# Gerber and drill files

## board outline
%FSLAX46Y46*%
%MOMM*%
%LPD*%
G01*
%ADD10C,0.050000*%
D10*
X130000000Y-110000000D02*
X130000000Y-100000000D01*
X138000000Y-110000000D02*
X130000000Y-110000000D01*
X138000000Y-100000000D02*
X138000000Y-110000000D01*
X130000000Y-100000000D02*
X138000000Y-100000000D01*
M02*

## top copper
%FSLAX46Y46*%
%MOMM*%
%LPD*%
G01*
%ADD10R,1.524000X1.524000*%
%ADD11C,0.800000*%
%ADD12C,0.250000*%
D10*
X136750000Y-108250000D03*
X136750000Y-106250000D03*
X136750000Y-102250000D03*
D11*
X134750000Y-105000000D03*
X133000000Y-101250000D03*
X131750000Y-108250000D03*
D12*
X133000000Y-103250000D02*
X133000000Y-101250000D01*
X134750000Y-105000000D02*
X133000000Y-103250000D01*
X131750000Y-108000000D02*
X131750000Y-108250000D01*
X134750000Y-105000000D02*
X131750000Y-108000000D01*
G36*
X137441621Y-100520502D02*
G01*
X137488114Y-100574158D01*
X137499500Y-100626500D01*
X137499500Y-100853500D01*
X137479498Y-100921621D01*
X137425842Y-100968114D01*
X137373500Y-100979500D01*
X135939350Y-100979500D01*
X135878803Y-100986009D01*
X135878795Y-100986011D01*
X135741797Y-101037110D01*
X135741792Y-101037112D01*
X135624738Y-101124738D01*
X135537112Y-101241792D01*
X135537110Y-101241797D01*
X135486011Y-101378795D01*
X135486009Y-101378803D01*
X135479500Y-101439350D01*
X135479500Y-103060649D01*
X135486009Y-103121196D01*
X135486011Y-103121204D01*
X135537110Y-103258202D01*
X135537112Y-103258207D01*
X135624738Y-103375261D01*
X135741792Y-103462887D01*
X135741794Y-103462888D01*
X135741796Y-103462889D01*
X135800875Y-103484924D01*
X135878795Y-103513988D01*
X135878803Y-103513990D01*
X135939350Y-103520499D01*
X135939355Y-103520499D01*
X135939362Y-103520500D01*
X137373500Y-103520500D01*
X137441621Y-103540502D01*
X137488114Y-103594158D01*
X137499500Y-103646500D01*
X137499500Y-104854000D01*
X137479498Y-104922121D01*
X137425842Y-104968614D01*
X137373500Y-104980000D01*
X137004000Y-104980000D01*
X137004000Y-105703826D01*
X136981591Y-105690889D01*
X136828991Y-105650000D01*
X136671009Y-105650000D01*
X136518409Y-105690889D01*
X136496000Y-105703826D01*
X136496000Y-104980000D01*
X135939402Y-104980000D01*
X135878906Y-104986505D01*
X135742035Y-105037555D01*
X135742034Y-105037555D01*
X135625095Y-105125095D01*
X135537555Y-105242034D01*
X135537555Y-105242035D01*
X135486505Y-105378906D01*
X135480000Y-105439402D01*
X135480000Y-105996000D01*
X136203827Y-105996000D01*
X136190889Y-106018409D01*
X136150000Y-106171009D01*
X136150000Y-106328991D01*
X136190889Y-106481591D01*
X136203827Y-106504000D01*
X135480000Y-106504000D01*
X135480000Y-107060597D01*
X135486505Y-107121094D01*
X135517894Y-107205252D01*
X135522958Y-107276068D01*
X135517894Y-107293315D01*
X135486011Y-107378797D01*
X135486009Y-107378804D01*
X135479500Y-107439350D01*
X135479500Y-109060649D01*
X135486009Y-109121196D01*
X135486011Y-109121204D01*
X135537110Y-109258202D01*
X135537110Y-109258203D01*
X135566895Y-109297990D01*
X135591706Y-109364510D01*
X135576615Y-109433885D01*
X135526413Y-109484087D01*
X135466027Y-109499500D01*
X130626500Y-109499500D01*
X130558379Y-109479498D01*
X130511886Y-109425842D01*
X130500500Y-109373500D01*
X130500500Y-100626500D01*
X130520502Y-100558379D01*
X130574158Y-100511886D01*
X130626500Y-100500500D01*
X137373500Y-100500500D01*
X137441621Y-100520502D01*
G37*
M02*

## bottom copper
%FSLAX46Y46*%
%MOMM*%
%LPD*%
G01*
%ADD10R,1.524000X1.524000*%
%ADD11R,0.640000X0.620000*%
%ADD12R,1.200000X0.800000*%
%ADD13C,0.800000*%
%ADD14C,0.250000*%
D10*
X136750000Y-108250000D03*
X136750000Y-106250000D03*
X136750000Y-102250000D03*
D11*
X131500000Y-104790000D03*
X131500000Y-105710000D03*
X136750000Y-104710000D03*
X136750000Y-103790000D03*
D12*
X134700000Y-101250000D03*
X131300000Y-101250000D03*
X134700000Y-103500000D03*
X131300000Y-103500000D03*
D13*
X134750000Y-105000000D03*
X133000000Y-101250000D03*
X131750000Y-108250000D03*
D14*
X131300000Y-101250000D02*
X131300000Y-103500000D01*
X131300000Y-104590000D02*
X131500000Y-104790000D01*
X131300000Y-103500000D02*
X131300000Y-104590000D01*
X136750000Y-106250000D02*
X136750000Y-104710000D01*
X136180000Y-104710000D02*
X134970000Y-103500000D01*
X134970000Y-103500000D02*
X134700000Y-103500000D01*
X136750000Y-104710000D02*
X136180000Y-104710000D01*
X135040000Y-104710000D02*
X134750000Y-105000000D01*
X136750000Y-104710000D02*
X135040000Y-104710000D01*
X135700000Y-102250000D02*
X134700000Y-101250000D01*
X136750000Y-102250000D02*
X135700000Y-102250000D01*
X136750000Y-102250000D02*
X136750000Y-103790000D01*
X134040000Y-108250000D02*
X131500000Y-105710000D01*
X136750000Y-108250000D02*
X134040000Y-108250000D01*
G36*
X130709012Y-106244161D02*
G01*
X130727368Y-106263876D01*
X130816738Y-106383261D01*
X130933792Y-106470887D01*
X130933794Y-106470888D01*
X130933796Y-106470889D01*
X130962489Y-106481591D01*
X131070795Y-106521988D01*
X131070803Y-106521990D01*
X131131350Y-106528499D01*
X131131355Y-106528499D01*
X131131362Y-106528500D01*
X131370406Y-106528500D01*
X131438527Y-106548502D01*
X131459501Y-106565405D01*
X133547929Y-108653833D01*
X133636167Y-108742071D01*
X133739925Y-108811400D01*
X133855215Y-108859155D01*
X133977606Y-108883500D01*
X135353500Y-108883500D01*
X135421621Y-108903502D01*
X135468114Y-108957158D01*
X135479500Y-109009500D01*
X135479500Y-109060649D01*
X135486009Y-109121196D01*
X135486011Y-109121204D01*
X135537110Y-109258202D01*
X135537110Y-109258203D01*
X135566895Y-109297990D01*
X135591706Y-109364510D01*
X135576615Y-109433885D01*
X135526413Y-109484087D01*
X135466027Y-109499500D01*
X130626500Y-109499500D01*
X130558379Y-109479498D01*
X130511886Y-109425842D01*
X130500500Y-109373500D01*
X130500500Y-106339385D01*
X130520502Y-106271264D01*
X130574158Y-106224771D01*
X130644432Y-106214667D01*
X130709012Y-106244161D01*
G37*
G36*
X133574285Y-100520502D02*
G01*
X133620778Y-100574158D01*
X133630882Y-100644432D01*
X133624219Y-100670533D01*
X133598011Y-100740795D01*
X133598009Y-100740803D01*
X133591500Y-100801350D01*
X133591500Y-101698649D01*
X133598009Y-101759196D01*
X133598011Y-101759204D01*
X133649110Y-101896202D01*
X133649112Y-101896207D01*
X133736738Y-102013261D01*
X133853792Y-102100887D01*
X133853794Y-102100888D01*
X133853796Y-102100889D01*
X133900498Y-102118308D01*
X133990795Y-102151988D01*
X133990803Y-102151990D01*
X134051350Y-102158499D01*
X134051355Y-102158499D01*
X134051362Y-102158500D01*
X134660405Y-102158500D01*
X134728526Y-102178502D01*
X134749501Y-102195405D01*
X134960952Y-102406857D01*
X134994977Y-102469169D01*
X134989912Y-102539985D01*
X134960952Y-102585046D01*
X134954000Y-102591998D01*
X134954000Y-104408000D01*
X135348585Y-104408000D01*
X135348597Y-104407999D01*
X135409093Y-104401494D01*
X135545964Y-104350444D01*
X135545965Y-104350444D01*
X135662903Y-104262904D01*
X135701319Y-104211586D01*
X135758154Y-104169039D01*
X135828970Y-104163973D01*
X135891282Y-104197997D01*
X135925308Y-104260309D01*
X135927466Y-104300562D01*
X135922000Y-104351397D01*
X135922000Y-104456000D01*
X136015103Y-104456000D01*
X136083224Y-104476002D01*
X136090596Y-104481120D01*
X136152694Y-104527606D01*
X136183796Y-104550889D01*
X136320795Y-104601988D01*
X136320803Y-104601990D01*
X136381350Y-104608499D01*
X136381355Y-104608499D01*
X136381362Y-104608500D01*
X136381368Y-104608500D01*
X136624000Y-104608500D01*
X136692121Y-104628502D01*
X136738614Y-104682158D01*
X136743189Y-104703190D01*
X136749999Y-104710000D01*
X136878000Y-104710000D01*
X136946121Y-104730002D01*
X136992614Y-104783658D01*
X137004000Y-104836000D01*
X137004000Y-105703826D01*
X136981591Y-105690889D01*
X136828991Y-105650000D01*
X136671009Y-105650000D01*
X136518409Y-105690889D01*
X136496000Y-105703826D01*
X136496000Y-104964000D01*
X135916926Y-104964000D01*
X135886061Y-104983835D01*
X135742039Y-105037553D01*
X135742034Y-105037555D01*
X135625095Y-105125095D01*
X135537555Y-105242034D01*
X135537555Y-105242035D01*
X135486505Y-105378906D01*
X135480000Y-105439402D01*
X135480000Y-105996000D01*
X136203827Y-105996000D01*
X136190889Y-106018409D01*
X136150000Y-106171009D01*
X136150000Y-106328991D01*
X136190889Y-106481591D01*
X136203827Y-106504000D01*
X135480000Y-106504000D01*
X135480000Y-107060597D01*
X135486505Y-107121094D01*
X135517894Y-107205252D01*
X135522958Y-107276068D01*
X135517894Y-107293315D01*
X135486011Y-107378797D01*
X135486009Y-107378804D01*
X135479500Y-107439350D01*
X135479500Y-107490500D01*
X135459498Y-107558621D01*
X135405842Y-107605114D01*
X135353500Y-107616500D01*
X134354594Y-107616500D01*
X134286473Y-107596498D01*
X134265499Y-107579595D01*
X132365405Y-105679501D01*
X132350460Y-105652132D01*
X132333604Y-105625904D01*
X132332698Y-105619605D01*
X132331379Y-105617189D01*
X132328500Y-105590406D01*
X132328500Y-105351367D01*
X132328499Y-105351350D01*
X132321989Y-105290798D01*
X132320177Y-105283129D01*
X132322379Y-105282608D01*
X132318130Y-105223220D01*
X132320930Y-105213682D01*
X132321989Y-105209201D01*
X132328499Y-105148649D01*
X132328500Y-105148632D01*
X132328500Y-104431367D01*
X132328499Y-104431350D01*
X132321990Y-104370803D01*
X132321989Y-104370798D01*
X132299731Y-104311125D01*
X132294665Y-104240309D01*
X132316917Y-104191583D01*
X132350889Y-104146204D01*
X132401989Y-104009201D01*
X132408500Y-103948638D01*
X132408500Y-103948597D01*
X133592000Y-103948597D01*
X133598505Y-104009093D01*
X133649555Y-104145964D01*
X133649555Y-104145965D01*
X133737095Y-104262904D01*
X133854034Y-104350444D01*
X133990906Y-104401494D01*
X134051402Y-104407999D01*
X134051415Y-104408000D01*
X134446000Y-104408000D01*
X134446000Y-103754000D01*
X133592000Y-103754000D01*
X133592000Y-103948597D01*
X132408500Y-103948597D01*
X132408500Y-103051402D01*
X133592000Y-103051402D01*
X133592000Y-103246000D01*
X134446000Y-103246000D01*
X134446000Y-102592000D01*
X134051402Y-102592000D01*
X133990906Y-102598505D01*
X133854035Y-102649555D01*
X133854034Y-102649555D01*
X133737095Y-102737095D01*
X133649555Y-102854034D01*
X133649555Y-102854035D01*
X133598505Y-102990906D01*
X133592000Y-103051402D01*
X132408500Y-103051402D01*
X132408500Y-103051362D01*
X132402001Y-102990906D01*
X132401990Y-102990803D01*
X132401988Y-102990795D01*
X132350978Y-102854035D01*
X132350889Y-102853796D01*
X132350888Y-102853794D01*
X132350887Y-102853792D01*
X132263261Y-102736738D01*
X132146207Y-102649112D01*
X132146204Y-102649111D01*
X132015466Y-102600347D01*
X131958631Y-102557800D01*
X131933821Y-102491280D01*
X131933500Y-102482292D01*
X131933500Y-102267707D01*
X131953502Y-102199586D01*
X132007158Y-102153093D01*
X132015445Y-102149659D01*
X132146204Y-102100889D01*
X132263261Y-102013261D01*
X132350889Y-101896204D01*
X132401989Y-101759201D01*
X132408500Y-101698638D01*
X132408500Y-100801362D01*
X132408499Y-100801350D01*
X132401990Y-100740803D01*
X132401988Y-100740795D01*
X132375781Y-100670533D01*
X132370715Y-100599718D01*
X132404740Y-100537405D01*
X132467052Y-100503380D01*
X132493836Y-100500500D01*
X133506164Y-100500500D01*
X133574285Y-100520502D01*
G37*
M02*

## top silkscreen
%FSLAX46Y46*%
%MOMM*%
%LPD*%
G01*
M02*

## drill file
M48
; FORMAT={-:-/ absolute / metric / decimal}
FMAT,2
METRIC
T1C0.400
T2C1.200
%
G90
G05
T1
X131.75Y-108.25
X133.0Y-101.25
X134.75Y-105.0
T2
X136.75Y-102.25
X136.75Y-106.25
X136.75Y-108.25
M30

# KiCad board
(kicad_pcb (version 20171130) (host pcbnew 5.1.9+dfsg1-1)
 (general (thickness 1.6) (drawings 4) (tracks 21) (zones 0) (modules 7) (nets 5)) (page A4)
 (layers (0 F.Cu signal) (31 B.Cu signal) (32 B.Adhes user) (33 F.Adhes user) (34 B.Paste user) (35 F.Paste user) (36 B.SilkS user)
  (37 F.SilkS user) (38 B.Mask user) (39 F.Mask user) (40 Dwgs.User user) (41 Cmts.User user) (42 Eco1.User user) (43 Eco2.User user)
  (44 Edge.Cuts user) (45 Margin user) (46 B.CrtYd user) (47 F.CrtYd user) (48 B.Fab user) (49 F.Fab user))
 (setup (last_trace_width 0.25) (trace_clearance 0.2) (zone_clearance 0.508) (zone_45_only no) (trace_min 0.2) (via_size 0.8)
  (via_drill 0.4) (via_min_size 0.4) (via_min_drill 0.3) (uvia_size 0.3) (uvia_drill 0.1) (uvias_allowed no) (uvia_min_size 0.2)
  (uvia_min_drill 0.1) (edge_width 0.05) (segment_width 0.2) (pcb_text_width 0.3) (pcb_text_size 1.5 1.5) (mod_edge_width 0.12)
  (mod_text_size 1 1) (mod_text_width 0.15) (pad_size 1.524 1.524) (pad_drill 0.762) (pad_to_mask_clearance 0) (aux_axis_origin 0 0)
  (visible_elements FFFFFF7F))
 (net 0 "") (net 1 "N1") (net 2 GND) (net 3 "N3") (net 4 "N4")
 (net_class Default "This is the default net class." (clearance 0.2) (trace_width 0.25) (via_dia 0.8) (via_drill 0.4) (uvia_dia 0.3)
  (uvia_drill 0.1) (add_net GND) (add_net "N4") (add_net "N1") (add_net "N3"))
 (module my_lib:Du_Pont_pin (layer B.Cu) (at 136.75 108.25)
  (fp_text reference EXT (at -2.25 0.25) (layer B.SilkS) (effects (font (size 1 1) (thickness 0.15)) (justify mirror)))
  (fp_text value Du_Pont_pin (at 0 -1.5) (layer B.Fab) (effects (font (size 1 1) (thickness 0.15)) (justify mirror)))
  (pad 1 thru_hole rect (at 0 0) (size 1.524 1.524) (drill 1.2) (layers *.Cu *.Mask) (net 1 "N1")))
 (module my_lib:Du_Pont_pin (layer B.Cu) (at 136.75 106.25)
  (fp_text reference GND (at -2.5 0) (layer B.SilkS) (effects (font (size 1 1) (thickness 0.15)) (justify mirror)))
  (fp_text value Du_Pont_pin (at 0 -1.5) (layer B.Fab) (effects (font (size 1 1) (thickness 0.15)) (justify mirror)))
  (pad 1 thru_hole rect (at 0 0) (size 1.524 1.524) (drill 1.2) (layers *.Cu *.Mask) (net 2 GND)))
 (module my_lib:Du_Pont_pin (layer B.Cu) (at 136.75 102.25)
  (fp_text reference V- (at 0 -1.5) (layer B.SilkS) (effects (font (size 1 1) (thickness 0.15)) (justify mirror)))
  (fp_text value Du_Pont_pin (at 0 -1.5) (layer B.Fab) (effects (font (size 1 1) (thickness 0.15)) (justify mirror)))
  (pad 1 thru_hole rect (at 0 0) (size 1.524 1.524) (drill 1.2) (layers *.Cu *.Mask) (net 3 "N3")))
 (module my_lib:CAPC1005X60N (layer B.Cu) (at 131.5 105.25 270)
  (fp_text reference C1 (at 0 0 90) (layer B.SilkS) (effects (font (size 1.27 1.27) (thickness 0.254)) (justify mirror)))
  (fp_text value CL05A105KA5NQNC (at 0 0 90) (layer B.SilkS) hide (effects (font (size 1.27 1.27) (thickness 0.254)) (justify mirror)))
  (pad 1 smd rect (at -0.46 0 270) (size 0.62 0.64) (layers B.Cu B.Paste B.Mask) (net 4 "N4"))
  (pad 2 smd rect (at 0.46 0 270) (size 0.62 0.64) (layers B.Cu B.Paste B.Mask) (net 1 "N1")))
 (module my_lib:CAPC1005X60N (layer B.Cu) (at 136.75 104.25 270)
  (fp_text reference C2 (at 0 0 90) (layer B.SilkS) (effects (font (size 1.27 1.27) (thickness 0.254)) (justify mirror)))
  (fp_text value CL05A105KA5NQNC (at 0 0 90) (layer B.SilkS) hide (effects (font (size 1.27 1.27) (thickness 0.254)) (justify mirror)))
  (pad 2 smd rect (at 0.46 0 270) (size 0.62 0.64) (layers B.Cu B.Paste B.Mask) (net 2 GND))
  (pad 1 smd rect (at -0.46 0 270) (size 0.62 0.64) (layers B.Cu B.Paste B.Mask) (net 3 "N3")))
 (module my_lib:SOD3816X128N (layer B.Cu) (at 133 101.25)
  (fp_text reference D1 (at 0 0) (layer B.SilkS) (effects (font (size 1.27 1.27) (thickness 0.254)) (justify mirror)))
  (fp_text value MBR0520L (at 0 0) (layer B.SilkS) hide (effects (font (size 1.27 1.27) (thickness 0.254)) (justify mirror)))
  (pad 2 smd rect (at 1.7 0 270) (size 0.8 1.2) (layers B.Cu B.Paste B.Mask) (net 3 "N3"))
  (pad 1 smd rect (at -1.7 0 270) (size 0.8 1.2) (layers B.Cu B.Paste B.Mask) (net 4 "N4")))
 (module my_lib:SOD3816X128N (layer B.Cu) (at 133 103.5 180)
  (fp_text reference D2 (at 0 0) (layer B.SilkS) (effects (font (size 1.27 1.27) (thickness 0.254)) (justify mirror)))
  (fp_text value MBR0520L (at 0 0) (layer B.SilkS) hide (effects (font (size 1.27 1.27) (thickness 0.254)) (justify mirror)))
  (pad 1 smd rect (at -1.7 0 90) (size 0.8 1.2) (layers B.Cu B.Paste B.Mask) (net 2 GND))
  (pad 2 smd rect (at 1.7 0 90) (size 0.8 1.2) (layers B.Cu B.Paste B.Mask) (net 4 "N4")))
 (gr_line (start 130 110) (end 130 100) (layer Edge.Cuts) (width 0.05))
 (gr_line (start 138 110) (end 130 110) (layer Edge.Cuts) (width 0.05))
 (gr_line (start 138 100) (end 138 110) (layer Edge.Cuts) (width 0.05))
 (gr_line (start 130 100) (end 138 100) (layer Edge.Cuts) (width 0.05))
 (segment (start 131.3 101.25) (end 131.3 103.5) (width 0.25) (layer B.Cu) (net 4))
 (segment (start 131.3 104.59) (end 131.5 104.79) (width 0.25) (layer B.Cu) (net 4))
 (segment (start 131.3 103.5) (end 131.3 104.59) (width 0.25) (layer B.Cu) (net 4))
 (segment (start 136.75 106.25) (end 136.75 104.71) (width 0.25) (layer B.Cu) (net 2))
 (segment (start 136.18 104.71) (end 134.97 103.5) (width 0.25) (layer B.Cu) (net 2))
 (segment (start 134.97 103.5) (end 134.7 103.5) (width 0.25) (layer B.Cu) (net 2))
 (segment (start 136.75 104.71) (end 136.18 104.71) (width 0.25) (layer B.Cu) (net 2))
 (via (at 134.75 105) (size 0.8) (drill 0.4) (layers F.Cu B.Cu) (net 2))
 (segment (start 135.04 104.71) (end 134.75 105) (width 0.25) (layer B.Cu) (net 2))
 (segment (start 136.75 104.71) (end 135.04 104.71) (width 0.25) (layer B.Cu) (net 2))
 (via (at 133 101.25) (size 0.8) (drill 0.4) (layers F.Cu B.Cu) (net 2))
 (segment (start 133 103.25) (end 133 101.25) (width 0.25) (layer F.Cu) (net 2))
 (segment (start 134.75 105) (end 133 103.25) (width 0.25) (layer F.Cu) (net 2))
 (via (at 131.75 108.25) (size 0.8) (drill 0.4) (layers F.Cu B.Cu) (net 2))
 (segment (start 131.75 108) (end 131.75 108.25) (width 0.25) (layer F.Cu) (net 2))
 (segment (start 134.75 105) (end 131.75 108) (width 0.25) (layer F.Cu) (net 2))
 (segment (start 135.7 102.25) (end 134.7 101.25) (width 0.25) (layer B.Cu) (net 3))
 (segment (start 136.75 102.25) (end 135.7 102.25) (width 0.25) (layer B.Cu) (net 3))
 (segment (start 136.75 102.25) (end 136.75 103.79) (width 0.25) (layer B.Cu) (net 3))
 (segment (start 134.04 108.25) (end 131.5 105.71) (width 0.25) (layer B.Cu) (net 1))
 (segment (start 136.75 108.25) (end 134.04 108.25) (width 0.25) (layer B.Cu) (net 1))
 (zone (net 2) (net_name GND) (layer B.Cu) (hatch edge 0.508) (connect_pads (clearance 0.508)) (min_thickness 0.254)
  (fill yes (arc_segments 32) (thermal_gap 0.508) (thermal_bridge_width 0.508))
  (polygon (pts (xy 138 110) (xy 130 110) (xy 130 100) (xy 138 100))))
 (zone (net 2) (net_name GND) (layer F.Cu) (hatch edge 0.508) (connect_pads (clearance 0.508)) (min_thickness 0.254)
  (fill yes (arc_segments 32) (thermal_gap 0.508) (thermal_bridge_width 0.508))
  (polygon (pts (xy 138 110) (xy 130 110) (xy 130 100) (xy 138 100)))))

